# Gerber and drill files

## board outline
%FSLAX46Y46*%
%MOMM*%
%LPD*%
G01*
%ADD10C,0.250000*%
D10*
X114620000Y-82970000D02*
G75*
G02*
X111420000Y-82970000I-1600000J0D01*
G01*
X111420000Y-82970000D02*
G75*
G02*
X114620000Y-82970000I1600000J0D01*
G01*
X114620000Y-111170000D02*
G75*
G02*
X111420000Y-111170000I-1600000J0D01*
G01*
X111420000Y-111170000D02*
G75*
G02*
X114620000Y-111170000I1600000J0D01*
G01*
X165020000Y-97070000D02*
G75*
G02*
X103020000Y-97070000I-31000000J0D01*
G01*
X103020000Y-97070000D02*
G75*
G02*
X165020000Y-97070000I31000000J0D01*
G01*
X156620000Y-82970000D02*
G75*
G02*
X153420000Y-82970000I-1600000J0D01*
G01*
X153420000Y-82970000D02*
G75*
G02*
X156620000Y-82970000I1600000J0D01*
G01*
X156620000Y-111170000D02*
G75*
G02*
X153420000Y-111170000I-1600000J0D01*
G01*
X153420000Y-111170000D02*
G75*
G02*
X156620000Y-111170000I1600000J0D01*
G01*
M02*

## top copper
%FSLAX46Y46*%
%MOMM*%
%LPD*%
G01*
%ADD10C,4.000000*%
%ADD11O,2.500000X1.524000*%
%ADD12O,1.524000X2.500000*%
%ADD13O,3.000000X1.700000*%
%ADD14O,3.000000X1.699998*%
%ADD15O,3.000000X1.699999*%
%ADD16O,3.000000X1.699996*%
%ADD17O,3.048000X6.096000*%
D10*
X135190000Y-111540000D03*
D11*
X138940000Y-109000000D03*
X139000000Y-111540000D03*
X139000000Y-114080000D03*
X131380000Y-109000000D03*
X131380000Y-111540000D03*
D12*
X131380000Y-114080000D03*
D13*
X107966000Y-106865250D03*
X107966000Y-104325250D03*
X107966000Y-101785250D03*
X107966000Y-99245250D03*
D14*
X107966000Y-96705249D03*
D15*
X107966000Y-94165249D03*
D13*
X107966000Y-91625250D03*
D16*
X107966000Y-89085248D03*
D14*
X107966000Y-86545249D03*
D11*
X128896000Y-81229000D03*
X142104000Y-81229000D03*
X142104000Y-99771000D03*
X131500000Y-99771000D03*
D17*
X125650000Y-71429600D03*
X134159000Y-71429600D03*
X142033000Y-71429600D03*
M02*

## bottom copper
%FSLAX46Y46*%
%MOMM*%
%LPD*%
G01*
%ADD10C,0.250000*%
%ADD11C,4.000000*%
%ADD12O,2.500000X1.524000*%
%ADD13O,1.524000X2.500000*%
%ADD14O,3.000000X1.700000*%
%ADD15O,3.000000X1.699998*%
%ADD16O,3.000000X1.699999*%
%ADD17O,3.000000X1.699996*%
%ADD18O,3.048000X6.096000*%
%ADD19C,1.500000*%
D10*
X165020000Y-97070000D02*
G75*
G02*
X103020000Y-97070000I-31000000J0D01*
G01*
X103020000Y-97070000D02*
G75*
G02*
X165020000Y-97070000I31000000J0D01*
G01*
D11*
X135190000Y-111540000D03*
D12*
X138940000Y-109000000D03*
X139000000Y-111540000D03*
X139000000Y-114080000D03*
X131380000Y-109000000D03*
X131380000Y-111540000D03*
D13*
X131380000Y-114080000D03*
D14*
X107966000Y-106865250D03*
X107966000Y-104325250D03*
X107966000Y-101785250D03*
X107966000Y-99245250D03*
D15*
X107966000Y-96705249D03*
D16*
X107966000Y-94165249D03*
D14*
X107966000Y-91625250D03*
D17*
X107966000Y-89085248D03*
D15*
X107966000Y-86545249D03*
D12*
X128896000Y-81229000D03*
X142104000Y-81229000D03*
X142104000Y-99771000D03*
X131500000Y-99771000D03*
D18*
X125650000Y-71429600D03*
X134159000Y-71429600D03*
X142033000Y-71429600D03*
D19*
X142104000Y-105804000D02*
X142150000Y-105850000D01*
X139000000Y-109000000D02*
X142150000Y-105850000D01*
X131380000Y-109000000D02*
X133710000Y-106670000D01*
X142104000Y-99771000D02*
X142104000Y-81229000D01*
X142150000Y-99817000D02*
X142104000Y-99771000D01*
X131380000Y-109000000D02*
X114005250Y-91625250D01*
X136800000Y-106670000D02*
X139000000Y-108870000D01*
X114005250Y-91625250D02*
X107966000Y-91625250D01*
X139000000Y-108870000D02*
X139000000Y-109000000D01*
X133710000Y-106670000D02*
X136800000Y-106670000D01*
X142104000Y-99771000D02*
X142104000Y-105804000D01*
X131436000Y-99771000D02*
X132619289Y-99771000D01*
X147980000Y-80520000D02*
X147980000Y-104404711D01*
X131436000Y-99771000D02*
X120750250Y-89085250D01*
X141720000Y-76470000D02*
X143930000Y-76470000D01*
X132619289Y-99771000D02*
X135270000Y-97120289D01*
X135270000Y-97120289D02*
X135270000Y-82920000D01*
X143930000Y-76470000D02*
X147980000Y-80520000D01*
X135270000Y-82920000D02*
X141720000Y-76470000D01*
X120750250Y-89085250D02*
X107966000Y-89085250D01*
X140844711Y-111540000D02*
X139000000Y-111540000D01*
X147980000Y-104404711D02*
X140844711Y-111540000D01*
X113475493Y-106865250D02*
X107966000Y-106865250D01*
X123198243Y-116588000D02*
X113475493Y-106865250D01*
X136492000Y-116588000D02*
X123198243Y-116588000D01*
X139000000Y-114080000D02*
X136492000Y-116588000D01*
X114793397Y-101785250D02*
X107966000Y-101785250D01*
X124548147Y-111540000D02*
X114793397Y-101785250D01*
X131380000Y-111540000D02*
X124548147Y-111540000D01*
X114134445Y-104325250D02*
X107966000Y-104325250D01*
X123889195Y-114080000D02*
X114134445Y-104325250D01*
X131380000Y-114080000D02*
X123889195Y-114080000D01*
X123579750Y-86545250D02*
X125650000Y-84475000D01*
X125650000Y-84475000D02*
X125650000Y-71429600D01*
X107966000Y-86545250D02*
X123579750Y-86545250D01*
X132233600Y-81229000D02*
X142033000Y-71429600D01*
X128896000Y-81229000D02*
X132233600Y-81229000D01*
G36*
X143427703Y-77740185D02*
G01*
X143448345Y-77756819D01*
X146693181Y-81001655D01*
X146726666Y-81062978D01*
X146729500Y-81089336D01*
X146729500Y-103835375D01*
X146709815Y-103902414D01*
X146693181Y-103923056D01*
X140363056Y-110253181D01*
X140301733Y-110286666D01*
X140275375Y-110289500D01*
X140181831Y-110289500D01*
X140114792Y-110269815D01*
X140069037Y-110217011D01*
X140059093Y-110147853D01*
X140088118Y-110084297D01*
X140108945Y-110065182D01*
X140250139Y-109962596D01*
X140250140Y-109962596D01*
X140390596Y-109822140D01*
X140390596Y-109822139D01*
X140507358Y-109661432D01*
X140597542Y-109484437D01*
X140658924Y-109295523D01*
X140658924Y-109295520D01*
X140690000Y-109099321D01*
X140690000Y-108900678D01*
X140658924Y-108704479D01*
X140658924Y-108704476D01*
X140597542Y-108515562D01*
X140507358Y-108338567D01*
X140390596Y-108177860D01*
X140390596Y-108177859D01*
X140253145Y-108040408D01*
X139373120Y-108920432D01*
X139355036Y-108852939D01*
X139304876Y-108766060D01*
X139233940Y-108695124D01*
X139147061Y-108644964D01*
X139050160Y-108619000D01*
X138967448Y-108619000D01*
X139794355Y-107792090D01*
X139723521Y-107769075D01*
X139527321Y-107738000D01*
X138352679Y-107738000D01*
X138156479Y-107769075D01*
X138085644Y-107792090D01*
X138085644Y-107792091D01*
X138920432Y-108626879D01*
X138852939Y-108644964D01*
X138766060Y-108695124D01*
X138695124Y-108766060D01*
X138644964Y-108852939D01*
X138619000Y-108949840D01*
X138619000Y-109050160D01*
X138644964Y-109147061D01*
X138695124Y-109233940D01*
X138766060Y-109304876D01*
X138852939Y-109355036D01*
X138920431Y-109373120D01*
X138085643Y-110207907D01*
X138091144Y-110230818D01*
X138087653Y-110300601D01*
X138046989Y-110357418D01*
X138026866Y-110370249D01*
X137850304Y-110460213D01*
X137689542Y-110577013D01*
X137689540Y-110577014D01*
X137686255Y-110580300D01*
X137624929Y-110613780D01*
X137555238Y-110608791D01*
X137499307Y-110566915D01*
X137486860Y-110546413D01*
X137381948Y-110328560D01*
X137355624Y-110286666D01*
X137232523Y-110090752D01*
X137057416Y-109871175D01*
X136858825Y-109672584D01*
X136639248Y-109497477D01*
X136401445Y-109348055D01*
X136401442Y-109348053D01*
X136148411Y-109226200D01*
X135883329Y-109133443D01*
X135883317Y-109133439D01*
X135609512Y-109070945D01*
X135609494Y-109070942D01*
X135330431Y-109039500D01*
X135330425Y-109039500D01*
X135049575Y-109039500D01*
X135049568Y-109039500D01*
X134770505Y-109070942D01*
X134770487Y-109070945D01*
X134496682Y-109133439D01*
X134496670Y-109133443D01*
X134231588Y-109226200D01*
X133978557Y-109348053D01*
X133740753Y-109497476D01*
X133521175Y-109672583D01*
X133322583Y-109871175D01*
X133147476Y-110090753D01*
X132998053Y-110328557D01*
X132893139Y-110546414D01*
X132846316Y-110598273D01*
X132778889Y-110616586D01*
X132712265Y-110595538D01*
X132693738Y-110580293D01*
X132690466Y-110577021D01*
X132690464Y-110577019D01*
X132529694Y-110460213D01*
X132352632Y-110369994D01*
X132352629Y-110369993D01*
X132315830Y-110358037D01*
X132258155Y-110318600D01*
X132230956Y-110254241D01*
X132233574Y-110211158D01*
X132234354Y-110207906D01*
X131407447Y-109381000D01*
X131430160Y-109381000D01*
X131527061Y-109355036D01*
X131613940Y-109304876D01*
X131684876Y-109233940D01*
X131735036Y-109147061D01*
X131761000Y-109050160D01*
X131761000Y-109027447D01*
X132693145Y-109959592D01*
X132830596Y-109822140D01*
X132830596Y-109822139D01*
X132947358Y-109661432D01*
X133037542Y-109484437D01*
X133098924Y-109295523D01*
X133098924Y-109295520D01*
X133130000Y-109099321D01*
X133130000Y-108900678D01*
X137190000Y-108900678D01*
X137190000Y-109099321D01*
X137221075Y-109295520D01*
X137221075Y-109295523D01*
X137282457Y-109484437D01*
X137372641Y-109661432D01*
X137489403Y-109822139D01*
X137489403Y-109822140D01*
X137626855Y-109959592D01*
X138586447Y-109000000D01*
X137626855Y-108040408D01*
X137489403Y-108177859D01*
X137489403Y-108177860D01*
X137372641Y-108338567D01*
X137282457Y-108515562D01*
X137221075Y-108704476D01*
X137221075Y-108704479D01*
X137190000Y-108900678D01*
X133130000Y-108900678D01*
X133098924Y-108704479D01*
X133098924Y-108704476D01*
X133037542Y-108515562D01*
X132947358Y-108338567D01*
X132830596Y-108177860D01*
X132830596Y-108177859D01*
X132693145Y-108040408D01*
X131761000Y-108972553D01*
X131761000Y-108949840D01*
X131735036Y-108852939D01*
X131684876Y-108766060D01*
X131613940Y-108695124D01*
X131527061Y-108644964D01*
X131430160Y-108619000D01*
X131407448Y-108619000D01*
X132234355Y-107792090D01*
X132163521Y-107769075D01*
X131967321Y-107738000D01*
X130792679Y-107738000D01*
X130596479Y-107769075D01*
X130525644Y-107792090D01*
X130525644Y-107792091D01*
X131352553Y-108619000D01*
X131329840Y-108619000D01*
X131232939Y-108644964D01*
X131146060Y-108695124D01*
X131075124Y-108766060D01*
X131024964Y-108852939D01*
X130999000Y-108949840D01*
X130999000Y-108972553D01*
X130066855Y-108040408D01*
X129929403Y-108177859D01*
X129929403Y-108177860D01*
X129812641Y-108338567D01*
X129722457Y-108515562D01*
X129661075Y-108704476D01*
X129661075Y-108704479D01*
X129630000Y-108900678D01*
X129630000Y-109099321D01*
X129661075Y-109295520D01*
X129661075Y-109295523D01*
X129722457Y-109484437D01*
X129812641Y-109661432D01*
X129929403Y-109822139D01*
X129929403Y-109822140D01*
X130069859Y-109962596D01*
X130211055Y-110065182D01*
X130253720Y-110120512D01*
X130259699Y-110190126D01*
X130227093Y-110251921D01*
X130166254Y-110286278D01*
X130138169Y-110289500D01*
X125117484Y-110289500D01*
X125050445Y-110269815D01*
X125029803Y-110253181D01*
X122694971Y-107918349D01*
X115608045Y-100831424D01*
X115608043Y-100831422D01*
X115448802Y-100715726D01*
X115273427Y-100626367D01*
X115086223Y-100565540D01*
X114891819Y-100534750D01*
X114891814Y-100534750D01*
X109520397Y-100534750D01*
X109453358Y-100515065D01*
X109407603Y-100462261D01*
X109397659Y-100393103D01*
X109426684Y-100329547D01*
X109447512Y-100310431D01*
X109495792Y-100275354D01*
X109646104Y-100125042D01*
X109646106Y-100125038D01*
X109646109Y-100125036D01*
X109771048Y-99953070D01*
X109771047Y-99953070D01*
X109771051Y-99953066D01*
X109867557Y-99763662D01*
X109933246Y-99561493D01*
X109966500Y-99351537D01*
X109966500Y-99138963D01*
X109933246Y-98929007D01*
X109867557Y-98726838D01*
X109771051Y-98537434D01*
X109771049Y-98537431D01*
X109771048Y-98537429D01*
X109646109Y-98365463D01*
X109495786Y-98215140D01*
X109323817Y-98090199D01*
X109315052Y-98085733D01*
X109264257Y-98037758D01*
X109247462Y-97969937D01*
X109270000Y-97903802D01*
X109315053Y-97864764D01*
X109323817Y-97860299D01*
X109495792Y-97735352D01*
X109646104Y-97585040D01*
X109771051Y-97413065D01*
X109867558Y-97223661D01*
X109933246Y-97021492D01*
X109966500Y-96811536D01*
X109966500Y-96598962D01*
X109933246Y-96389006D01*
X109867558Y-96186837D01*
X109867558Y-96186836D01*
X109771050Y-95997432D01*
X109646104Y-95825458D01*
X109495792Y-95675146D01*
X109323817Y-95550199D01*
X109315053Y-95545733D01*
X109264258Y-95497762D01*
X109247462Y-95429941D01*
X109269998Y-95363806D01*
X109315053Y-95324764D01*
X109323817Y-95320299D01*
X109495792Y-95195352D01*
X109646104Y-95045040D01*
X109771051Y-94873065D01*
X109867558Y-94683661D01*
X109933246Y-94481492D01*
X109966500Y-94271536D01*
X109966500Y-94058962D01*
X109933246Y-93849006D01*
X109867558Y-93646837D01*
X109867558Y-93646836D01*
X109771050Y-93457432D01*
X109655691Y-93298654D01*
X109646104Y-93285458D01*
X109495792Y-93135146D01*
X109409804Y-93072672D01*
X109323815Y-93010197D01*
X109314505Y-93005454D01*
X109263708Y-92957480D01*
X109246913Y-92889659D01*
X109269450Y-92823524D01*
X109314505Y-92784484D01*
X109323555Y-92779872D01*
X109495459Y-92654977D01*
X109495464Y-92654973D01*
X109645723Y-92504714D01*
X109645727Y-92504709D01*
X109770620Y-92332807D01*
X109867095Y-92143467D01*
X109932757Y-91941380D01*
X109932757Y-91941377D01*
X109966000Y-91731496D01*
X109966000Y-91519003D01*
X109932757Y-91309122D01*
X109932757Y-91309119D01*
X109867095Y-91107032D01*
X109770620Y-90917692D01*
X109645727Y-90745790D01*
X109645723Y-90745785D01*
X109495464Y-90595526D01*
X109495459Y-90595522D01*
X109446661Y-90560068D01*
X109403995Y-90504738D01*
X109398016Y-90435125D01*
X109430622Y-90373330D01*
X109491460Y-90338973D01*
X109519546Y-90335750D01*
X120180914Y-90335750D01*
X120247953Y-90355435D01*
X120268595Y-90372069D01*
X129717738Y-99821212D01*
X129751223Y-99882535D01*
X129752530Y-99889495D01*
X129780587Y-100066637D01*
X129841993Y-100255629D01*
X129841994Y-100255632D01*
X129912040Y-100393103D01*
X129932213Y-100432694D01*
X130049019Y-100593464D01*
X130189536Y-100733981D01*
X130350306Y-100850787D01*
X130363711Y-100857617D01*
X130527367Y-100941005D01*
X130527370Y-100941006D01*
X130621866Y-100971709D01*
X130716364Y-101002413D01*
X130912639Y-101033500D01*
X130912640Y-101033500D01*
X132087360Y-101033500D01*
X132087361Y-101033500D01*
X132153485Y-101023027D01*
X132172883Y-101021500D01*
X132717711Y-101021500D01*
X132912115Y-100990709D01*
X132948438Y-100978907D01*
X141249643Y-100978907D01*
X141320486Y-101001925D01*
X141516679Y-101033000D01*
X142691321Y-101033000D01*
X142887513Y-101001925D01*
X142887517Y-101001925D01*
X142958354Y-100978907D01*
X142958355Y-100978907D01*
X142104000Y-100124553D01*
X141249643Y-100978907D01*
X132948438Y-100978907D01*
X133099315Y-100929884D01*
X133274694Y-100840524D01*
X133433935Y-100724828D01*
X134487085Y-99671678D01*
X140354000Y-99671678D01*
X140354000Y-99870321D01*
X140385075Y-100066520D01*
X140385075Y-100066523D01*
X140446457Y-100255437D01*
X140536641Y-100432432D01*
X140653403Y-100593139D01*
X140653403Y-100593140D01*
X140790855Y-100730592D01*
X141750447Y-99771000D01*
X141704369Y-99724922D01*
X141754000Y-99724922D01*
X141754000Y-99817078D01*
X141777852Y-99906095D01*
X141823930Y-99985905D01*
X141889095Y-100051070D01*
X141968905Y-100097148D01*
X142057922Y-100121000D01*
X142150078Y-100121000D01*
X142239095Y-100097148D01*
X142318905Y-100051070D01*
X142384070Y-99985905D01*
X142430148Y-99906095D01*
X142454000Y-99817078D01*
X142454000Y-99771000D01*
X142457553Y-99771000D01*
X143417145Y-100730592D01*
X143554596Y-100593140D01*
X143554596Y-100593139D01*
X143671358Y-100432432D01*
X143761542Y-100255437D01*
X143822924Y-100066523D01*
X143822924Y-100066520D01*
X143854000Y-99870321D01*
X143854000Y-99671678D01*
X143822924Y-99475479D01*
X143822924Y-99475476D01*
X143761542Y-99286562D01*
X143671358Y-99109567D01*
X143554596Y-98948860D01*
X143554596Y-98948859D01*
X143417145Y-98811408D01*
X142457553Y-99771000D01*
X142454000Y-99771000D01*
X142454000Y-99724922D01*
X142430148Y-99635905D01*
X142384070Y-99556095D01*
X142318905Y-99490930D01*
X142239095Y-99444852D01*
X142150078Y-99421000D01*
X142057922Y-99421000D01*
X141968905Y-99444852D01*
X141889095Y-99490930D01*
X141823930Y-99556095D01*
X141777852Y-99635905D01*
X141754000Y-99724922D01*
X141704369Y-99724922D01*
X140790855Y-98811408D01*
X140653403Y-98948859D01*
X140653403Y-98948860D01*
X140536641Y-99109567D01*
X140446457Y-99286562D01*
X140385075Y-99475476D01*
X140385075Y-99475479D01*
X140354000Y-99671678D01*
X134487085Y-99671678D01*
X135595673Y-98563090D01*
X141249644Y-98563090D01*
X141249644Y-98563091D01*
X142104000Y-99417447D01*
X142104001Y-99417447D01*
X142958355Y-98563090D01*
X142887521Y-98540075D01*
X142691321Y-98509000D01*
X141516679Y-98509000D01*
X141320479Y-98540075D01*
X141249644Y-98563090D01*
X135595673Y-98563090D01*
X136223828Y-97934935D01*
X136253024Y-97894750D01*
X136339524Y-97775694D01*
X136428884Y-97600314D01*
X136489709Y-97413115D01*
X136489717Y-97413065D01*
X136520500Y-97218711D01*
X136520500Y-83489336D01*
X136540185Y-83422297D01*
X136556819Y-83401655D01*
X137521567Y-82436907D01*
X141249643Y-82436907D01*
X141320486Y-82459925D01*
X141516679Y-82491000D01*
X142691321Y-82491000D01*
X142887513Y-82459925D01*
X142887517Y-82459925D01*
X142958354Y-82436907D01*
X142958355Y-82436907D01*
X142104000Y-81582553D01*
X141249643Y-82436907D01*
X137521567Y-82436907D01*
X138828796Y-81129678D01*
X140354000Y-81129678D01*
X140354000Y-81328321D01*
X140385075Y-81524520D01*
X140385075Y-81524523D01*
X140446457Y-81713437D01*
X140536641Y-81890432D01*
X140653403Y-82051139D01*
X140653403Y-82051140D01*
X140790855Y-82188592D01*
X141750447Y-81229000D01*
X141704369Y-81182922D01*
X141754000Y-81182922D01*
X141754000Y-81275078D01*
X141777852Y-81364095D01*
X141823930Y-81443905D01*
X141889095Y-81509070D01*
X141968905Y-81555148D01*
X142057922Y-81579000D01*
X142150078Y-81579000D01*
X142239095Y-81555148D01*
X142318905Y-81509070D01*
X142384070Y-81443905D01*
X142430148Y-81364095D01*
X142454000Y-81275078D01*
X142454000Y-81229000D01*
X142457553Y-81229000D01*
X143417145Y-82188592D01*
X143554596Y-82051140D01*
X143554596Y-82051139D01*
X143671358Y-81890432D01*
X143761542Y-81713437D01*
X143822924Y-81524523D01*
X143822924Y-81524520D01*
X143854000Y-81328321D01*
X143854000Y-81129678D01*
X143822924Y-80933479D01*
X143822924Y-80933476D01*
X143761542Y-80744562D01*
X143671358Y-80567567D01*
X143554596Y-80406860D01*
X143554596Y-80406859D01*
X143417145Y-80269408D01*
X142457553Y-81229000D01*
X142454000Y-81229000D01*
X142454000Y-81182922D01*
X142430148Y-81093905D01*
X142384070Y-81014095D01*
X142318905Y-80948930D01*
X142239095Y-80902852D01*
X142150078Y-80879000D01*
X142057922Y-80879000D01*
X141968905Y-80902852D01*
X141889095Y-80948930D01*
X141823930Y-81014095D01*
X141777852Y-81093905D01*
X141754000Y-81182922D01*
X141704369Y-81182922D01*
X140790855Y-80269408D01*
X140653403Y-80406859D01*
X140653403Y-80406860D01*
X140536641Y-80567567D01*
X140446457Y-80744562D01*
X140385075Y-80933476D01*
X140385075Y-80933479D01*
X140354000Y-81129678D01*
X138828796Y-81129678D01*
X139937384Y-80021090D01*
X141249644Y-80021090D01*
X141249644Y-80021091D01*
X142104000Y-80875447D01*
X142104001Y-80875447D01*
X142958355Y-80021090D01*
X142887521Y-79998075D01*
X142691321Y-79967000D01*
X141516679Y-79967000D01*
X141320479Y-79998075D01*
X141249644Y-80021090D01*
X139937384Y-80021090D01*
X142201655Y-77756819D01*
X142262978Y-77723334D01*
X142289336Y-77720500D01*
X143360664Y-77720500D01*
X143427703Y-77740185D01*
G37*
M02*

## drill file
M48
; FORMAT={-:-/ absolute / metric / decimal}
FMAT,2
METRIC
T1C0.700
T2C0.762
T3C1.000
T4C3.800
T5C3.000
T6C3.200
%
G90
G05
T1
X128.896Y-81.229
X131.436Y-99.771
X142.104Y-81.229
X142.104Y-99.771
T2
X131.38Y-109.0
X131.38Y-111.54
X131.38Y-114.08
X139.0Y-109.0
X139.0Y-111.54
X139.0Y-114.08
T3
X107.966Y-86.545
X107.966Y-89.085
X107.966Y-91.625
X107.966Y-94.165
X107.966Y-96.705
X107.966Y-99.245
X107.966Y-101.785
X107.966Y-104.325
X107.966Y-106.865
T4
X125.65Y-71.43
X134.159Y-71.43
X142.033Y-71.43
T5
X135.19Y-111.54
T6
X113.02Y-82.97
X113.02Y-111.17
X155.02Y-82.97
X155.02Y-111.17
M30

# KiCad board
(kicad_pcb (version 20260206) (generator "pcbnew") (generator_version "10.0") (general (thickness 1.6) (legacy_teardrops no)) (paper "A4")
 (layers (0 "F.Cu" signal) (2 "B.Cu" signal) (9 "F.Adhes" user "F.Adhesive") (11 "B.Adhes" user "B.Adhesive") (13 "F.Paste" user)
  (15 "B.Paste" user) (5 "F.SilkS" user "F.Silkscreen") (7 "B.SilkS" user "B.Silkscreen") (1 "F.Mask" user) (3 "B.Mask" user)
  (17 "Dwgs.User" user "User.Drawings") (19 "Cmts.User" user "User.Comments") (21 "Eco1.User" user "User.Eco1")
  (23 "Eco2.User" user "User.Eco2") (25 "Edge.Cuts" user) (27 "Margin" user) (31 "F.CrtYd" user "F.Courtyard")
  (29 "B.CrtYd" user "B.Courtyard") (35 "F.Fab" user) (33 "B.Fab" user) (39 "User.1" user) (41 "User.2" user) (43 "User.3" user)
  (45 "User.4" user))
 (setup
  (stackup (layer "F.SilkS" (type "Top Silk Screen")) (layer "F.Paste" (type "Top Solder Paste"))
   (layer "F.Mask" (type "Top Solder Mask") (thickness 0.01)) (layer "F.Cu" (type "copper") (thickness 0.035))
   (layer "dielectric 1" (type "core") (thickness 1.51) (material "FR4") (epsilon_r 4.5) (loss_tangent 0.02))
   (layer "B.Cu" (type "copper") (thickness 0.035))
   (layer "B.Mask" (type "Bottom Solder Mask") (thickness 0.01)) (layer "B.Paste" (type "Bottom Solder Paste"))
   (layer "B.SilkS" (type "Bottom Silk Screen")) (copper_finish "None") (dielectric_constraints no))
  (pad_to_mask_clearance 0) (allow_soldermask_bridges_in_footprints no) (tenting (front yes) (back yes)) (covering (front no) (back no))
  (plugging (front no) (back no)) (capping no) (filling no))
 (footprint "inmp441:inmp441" (layer "F.Cu") (at 135.19 111.54 -90)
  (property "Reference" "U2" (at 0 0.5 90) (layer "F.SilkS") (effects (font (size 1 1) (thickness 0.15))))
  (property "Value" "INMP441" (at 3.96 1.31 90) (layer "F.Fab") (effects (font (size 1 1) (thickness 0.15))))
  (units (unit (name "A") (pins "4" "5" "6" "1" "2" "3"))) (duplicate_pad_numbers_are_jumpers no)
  (pad "" np_thru_hole circle (at 0 0 270) (size 4 4) (drill 3) (layers "*.Cu" "*.Mask"))
  (pad "1" thru_hole oval (at -2.54 -3.81 270) (size 1.524 2.5) (drill 0.762 (offset 0 0.06)) (layers "*.Cu" "*.Mask")
   (remove_unused_layers no) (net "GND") (thermal_bridge_angle 45))
  (pad "2" thru_hole oval (at 0 -3.81 270) (size 1.524 2.5) (drill 0.762) (layers "*.Cu" "*.Mask") (remove_unused_layers no) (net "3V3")
   (thermal_bridge_angle 45))
  (pad "3" thru_hole oval (at 2.54 -3.81 270) (size 1.524 2.5) (drill 0.762) (layers "*.Cu" "*.Mask") (remove_unused_layers no)
   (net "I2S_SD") (thermal_bridge_angle 45))
  (pad "4" thru_hole oval (at -2.54 3.81 270) (size 1.524 2.5) (drill 0.762) (layers "*.Cu" "*.Mask") (remove_unused_layers no) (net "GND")
   (thermal_bridge_angle 45))
  (pad "5" thru_hole oval (at 0 3.81 270) (size 1.524 2.5) (drill 0.762) (layers "*.Cu" "*.Mask") (remove_unused_layers no) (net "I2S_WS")
   (thermal_bridge_angle 45))
  (pad "6" thru_hole oval (at 2.54 3.81) (size 1.524 2.5) (drill 0.762) (layers "*.Cu" "*.Mask") (remove_unused_layers no) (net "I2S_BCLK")
   (thermal_bridge_angle 45)))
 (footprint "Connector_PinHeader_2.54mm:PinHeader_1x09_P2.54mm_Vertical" (layer "F.Cu") (at 107.966 106.86525 180)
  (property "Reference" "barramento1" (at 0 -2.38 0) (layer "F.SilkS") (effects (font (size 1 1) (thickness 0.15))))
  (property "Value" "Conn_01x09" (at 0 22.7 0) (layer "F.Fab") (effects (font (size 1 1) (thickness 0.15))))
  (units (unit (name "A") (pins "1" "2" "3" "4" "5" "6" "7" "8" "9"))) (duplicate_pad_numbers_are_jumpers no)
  (pad "1" thru_hole oval (at 0 0 180) (size 3 1.7) (drill 1) (layers "*.Cu" "*.Mask") (remove_unused_layers no) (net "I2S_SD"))
  (pad "2" thru_hole oval (at 0 2.54 180) (size 3 1.7) (drill 1) (layers "*.Cu" "*.Mask") (remove_unused_layers no) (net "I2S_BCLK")
   (thermal_bridge_angle 45))
  (pad "3" thru_hole oval (at 0 5.08 180) (size 3 1.7) (drill 1) (layers "*.Cu" "*.Mask") (remove_unused_layers no) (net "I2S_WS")
   (thermal_bridge_angle 45))
  (pad "4" thru_hole oval (at 0 7.62 180) (size 3 1.7) (drill 1) (layers "*.Cu" "*.Mask") (remove_unused_layers no) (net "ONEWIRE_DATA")
   (thermal_bridge_angle 45))
  (pad "5" thru_hole oval (at 0 10.16 180) (size 3 1.699998) (drill 1 (offset 0 0.000001)) (layers "*.Cu" "*.Mask")
   (remove_unused_layers no) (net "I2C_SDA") (thermal_bridge_angle 45))
  (pad "6" thru_hole oval (at 0 12.7 180) (size 3 1.699999) (drill 1 (offset 0 0.000001)) (layers "*.Cu" "*.Mask") (remove_unused_layers no)
   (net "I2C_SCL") (thermal_bridge_angle 45))
  (pad "7" thru_hole oval (at 0 15.24 180) (size 3 1.7) (drill 1) (layers "*.Cu" "*.Mask") (remove_unused_layers no) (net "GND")
   (thermal_bridge_angle 45))
  (pad "8" thru_hole oval (at 0 17.78 180) (size 3 1.699996) (drill 1 (offset 0 0.000002)) (layers "*.Cu" "*.Mask")
   (remove_unused_layers no) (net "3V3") (thermal_bridge_angle 45))
  (pad "9" thru_hole oval (at 0 20.32 180) (size 3 1.699998) (drill 1 (offset 0 0.000001)) (layers "*.Cu" "*.Mask")
   (remove_unused_layers no) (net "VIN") (thermal_bridge_angle 45)))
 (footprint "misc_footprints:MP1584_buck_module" (layer "F.Cu") (at 135.5 90.5 -90)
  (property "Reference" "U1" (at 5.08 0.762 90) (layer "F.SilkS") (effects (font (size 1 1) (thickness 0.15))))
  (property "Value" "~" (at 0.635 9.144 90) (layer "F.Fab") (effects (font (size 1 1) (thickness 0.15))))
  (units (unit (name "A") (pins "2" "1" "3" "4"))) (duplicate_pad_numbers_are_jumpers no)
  (pad "1" thru_hole oval (at -9.271 6.604 270) (size 1.524 2.5) (drill 0.7) (layers "*.Cu" "*.Mask" "F.SilkS") (remove_unused_layers no)
   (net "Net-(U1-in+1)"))
  (pad "2" thru_hole oval (at -9.271 -6.604 270) (size 1.524 2.5) (drill 0.7) (layers "*.Cu" "*.Mask" "F.SilkS") (remove_unused_layers no)
   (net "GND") (thermal_bridge_angle 45))
  (pad "3" thru_hole oval (at 9.271 -6.604 270) (size 1.524 2.5) (drill 0.7) (layers "*.Cu" "*.Mask" "F.SilkS") (remove_unused_layers no)
   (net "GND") (thermal_bridge_angle 45))
  (pad "4" thru_hole oval (at 9.271 4.064 270) (size 1.524 2.5) (drill 0.7 (offset 0 -0.064)) (layers "*.Cu" "*.Mask" "F.SilkS")
   (remove_unused_layers no) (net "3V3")))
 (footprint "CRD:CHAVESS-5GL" (layer "F.Cu") (at 134.794 72.1916)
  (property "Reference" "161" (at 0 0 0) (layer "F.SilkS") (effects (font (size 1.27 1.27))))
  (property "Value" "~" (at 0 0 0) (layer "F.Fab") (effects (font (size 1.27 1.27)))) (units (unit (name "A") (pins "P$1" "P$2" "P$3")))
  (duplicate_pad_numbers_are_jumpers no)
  (pad "P$1" thru_hole oval (at -9.144 -0.762 90) (size 6.096 3.048) (drill 3.8) (layers "*.Cu" "*.Mask") (remove_unused_layers no)
   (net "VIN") (solder_mask_margin 0.1016) (thermal_bridge_angle 0))
  (pad "P$2" thru_hole oval (at -0.635 -0.762 90) (size 6.096 3.048) (drill 3.8) (layers "*.Cu" "*.Mask") (remove_unused_layers no)
   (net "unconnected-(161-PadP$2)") (solder_mask_margin 0.1016) (thermal_bridge_angle 0))
  (pad "P$3" thru_hole oval (at 7.239 -0.762 90) (size 6.096 3.048) (drill 3.8) (layers "*.Cu" "*.Mask") (remove_unused_layers no)
   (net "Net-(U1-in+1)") (solder_mask_margin 0.1016) (thermal_bridge_angle 0)))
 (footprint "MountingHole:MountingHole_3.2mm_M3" (layer "F.Cu") (at 113.02 82.97)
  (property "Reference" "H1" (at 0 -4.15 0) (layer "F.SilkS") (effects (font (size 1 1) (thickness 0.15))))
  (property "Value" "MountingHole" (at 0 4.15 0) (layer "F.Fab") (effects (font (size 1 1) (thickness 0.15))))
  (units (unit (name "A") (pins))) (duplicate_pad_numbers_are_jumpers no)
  (pad "" np_thru_hole circle (at 0 0) (size 3.2 3.2) (drill 3.2) (layers "*.Cu" "*.Mask")))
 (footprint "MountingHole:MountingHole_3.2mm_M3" (layer "F.Cu") (at 113.02 111.17)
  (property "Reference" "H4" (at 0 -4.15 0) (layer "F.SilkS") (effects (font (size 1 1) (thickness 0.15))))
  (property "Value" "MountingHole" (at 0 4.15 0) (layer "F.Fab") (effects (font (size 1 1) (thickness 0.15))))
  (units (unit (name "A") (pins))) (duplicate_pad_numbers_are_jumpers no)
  (pad "" np_thru_hole circle (at 0 0) (size 3.2 3.2) (drill 3.2) (layers "*.Cu" "*.Mask")))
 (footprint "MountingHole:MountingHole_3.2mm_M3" (layer "F.Cu") (at 155.02 111.17)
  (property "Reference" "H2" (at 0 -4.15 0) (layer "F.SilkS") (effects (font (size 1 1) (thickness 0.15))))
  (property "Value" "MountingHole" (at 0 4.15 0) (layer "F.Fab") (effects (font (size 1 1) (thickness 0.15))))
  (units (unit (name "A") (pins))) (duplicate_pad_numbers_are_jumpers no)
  (pad "" np_thru_hole circle (at 0 0) (size 3.2 3.2) (drill 3.2) (layers "*.Cu" "*.Mask")))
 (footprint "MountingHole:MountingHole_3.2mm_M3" (layer "F.Cu") (at 155.02 82.97)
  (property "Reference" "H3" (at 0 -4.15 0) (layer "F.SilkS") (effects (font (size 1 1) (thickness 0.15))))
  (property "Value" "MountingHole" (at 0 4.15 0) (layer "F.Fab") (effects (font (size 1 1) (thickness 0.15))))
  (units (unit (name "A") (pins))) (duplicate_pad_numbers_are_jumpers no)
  (pad "" np_thru_hole circle (at 0 0) (size 3.2 3.2) (drill 3.2) (layers "*.Cu" "*.Mask")))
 (gr_circle (center 134.02 97.07) (end 165.02 97.07) (stroke (width 0.25) (type solid)) (fill no) (layer "B.Cu"))
 (gr_circle (center 113.02 82.97) (end 114.62 82.97) (stroke (width 0.25) (type default)) (fill no) (layer "Edge.Cuts"))
 (gr_circle (center 113.02 111.17) (end 114.62 111.17) (stroke (width 0.25) (type default)) (fill no) (layer "Edge.Cuts"))
 (gr_circle (center 134.02 97.07) (end 165.02 97.07) (stroke (width 0.25) (type solid)) (fill no) (layer "Edge.Cuts"))
 (gr_circle (center 155.02 82.97) (end 156.62 82.97) (stroke (width 0.25) (type default)) (fill no) (layer "Edge.Cuts"))
 (gr_circle (center 155.02 111.17) (end 156.62 111.17) (stroke (width 0.25) (type default)) (fill no) (layer "Edge.Cuts"))
 (segment (start 142.104 105.804) (end 142.15 105.85) (width 1.5) (layer "B.Cu") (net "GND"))
 (segment (start 139 109) (end 142.15 105.85) (width 1.5) (layer "B.Cu") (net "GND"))
 (segment (start 131.38 109) (end 133.71 106.67) (width 1.5) (layer "B.Cu") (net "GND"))
 (segment (start 142.104 99.771) (end 142.104 81.229) (width 1.5) (layer "B.Cu") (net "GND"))
 (segment (start 142.15 99.817) (end 142.104 99.771) (width 1.5) (layer "B.Cu") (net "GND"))
 (segment (start 131.38 109) (end 114.00525 91.62525) (width 1.5) (layer "B.Cu") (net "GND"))
 (segment (start 136.8 106.67) (end 139 108.87) (width 1.5) (layer "B.Cu") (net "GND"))
 (segment (start 114.00525 91.62525) (end 107.966 91.62525) (width 1.5) (layer "B.Cu") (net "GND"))
 (segment (start 139 108.87) (end 139 109) (width 1.5) (layer "B.Cu") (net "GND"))
 (segment (start 133.71 106.67) (end 136.8 106.67) (width 1.5) (layer "B.Cu") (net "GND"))
 (segment (start 142.104 99.771) (end 142.104 105.804) (width 1.5) (layer "B.Cu") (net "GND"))
 (segment (start 131.436 99.771) (end 132.619289 99.771) (width 1.5) (layer "B.Cu") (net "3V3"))
 (segment (start 147.98 80.52) (end 147.98 104.404711) (width 1.5) (layer "B.Cu") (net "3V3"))
 (segment (start 131.436 99.771) (end 120.75025 89.08525) (width 1.5) (layer "B.Cu") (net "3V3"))
 (segment (start 141.72 76.47) (end 143.93 76.47) (width 1.5) (layer "B.Cu") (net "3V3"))
 (segment (start 132.619289 99.771) (end 135.27 97.120289) (width 1.5) (layer "B.Cu") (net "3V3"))
 (segment (start 135.27 97.120289) (end 135.27 82.92) (width 1.5) (layer "B.Cu") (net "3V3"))
 (segment (start 143.93 76.47) (end 147.98 80.52) (width 1.5) (layer "B.Cu") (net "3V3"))
 (segment (start 135.27 82.92) (end 141.72 76.47) (width 1.5) (layer "B.Cu") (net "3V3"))
 (segment (start 120.75025 89.08525) (end 107.966 89.08525) (width 1.5) (layer "B.Cu") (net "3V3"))
 (segment (start 140.844711 111.54) (end 139 111.54) (width 1.5) (layer "B.Cu") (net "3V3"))
 (segment (start 147.98 104.404711) (end 140.844711 111.54) (width 1.5) (layer "B.Cu") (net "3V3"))
 (segment (start 113.475493 106.86525) (end 107.966 106.86525) (width 1.5) (layer "B.Cu") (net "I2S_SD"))
 (segment (start 123.198243 116.588) (end 113.475493 106.86525) (width 1.5) (layer "B.Cu") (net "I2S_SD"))
 (segment (start 136.492 116.588) (end 123.198243 116.588) (width 1.5) (layer "B.Cu") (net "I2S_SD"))
 (segment (start 139 114.08) (end 136.492 116.588) (width 1.5) (layer "B.Cu") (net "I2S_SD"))
 (segment (start 114.793397 101.78525) (end 107.966 101.78525) (width 1.5) (layer "B.Cu") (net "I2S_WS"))
 (segment (start 124.548147 111.54) (end 114.793397 101.78525) (width 1.5) (layer "B.Cu") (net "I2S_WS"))
 (segment (start 131.38 111.54) (end 124.548147 111.54) (width 1.5) (layer "B.Cu") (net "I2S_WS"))
 (segment (start 114.134445 104.32525) (end 107.966 104.32525) (width 1.5) (layer "B.Cu") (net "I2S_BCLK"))
 (segment (start 123.889195 114.08) (end 114.134445 104.32525) (width 1.5) (layer "B.Cu") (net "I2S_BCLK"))
 (segment (start 131.38 114.08) (end 123.889195 114.08) (width 1.5) (layer "B.Cu") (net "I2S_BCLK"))
 (segment (start 123.57975 86.54525) (end 125.65 84.475) (width 1.5) (layer "B.Cu") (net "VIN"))
 (segment (start 125.65 84.475) (end 125.65 71.4296) (width 1.5) (layer "B.Cu") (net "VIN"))
 (segment (start 107.966 86.54525) (end 123.57975 86.54525) (width 1.5) (layer "B.Cu") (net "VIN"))
 (segment (start 132.2336 81.229) (end 142.033 71.4296) (width 1.5) (layer "B.Cu") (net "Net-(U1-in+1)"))
 (segment (start 128.896 81.229) (end 132.2336 81.229) (width 1.5) (layer "B.Cu") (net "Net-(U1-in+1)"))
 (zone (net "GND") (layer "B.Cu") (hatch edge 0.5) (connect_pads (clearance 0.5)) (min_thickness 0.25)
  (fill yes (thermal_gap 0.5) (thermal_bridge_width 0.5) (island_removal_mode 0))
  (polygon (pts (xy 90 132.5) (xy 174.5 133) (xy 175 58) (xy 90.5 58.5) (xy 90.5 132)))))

